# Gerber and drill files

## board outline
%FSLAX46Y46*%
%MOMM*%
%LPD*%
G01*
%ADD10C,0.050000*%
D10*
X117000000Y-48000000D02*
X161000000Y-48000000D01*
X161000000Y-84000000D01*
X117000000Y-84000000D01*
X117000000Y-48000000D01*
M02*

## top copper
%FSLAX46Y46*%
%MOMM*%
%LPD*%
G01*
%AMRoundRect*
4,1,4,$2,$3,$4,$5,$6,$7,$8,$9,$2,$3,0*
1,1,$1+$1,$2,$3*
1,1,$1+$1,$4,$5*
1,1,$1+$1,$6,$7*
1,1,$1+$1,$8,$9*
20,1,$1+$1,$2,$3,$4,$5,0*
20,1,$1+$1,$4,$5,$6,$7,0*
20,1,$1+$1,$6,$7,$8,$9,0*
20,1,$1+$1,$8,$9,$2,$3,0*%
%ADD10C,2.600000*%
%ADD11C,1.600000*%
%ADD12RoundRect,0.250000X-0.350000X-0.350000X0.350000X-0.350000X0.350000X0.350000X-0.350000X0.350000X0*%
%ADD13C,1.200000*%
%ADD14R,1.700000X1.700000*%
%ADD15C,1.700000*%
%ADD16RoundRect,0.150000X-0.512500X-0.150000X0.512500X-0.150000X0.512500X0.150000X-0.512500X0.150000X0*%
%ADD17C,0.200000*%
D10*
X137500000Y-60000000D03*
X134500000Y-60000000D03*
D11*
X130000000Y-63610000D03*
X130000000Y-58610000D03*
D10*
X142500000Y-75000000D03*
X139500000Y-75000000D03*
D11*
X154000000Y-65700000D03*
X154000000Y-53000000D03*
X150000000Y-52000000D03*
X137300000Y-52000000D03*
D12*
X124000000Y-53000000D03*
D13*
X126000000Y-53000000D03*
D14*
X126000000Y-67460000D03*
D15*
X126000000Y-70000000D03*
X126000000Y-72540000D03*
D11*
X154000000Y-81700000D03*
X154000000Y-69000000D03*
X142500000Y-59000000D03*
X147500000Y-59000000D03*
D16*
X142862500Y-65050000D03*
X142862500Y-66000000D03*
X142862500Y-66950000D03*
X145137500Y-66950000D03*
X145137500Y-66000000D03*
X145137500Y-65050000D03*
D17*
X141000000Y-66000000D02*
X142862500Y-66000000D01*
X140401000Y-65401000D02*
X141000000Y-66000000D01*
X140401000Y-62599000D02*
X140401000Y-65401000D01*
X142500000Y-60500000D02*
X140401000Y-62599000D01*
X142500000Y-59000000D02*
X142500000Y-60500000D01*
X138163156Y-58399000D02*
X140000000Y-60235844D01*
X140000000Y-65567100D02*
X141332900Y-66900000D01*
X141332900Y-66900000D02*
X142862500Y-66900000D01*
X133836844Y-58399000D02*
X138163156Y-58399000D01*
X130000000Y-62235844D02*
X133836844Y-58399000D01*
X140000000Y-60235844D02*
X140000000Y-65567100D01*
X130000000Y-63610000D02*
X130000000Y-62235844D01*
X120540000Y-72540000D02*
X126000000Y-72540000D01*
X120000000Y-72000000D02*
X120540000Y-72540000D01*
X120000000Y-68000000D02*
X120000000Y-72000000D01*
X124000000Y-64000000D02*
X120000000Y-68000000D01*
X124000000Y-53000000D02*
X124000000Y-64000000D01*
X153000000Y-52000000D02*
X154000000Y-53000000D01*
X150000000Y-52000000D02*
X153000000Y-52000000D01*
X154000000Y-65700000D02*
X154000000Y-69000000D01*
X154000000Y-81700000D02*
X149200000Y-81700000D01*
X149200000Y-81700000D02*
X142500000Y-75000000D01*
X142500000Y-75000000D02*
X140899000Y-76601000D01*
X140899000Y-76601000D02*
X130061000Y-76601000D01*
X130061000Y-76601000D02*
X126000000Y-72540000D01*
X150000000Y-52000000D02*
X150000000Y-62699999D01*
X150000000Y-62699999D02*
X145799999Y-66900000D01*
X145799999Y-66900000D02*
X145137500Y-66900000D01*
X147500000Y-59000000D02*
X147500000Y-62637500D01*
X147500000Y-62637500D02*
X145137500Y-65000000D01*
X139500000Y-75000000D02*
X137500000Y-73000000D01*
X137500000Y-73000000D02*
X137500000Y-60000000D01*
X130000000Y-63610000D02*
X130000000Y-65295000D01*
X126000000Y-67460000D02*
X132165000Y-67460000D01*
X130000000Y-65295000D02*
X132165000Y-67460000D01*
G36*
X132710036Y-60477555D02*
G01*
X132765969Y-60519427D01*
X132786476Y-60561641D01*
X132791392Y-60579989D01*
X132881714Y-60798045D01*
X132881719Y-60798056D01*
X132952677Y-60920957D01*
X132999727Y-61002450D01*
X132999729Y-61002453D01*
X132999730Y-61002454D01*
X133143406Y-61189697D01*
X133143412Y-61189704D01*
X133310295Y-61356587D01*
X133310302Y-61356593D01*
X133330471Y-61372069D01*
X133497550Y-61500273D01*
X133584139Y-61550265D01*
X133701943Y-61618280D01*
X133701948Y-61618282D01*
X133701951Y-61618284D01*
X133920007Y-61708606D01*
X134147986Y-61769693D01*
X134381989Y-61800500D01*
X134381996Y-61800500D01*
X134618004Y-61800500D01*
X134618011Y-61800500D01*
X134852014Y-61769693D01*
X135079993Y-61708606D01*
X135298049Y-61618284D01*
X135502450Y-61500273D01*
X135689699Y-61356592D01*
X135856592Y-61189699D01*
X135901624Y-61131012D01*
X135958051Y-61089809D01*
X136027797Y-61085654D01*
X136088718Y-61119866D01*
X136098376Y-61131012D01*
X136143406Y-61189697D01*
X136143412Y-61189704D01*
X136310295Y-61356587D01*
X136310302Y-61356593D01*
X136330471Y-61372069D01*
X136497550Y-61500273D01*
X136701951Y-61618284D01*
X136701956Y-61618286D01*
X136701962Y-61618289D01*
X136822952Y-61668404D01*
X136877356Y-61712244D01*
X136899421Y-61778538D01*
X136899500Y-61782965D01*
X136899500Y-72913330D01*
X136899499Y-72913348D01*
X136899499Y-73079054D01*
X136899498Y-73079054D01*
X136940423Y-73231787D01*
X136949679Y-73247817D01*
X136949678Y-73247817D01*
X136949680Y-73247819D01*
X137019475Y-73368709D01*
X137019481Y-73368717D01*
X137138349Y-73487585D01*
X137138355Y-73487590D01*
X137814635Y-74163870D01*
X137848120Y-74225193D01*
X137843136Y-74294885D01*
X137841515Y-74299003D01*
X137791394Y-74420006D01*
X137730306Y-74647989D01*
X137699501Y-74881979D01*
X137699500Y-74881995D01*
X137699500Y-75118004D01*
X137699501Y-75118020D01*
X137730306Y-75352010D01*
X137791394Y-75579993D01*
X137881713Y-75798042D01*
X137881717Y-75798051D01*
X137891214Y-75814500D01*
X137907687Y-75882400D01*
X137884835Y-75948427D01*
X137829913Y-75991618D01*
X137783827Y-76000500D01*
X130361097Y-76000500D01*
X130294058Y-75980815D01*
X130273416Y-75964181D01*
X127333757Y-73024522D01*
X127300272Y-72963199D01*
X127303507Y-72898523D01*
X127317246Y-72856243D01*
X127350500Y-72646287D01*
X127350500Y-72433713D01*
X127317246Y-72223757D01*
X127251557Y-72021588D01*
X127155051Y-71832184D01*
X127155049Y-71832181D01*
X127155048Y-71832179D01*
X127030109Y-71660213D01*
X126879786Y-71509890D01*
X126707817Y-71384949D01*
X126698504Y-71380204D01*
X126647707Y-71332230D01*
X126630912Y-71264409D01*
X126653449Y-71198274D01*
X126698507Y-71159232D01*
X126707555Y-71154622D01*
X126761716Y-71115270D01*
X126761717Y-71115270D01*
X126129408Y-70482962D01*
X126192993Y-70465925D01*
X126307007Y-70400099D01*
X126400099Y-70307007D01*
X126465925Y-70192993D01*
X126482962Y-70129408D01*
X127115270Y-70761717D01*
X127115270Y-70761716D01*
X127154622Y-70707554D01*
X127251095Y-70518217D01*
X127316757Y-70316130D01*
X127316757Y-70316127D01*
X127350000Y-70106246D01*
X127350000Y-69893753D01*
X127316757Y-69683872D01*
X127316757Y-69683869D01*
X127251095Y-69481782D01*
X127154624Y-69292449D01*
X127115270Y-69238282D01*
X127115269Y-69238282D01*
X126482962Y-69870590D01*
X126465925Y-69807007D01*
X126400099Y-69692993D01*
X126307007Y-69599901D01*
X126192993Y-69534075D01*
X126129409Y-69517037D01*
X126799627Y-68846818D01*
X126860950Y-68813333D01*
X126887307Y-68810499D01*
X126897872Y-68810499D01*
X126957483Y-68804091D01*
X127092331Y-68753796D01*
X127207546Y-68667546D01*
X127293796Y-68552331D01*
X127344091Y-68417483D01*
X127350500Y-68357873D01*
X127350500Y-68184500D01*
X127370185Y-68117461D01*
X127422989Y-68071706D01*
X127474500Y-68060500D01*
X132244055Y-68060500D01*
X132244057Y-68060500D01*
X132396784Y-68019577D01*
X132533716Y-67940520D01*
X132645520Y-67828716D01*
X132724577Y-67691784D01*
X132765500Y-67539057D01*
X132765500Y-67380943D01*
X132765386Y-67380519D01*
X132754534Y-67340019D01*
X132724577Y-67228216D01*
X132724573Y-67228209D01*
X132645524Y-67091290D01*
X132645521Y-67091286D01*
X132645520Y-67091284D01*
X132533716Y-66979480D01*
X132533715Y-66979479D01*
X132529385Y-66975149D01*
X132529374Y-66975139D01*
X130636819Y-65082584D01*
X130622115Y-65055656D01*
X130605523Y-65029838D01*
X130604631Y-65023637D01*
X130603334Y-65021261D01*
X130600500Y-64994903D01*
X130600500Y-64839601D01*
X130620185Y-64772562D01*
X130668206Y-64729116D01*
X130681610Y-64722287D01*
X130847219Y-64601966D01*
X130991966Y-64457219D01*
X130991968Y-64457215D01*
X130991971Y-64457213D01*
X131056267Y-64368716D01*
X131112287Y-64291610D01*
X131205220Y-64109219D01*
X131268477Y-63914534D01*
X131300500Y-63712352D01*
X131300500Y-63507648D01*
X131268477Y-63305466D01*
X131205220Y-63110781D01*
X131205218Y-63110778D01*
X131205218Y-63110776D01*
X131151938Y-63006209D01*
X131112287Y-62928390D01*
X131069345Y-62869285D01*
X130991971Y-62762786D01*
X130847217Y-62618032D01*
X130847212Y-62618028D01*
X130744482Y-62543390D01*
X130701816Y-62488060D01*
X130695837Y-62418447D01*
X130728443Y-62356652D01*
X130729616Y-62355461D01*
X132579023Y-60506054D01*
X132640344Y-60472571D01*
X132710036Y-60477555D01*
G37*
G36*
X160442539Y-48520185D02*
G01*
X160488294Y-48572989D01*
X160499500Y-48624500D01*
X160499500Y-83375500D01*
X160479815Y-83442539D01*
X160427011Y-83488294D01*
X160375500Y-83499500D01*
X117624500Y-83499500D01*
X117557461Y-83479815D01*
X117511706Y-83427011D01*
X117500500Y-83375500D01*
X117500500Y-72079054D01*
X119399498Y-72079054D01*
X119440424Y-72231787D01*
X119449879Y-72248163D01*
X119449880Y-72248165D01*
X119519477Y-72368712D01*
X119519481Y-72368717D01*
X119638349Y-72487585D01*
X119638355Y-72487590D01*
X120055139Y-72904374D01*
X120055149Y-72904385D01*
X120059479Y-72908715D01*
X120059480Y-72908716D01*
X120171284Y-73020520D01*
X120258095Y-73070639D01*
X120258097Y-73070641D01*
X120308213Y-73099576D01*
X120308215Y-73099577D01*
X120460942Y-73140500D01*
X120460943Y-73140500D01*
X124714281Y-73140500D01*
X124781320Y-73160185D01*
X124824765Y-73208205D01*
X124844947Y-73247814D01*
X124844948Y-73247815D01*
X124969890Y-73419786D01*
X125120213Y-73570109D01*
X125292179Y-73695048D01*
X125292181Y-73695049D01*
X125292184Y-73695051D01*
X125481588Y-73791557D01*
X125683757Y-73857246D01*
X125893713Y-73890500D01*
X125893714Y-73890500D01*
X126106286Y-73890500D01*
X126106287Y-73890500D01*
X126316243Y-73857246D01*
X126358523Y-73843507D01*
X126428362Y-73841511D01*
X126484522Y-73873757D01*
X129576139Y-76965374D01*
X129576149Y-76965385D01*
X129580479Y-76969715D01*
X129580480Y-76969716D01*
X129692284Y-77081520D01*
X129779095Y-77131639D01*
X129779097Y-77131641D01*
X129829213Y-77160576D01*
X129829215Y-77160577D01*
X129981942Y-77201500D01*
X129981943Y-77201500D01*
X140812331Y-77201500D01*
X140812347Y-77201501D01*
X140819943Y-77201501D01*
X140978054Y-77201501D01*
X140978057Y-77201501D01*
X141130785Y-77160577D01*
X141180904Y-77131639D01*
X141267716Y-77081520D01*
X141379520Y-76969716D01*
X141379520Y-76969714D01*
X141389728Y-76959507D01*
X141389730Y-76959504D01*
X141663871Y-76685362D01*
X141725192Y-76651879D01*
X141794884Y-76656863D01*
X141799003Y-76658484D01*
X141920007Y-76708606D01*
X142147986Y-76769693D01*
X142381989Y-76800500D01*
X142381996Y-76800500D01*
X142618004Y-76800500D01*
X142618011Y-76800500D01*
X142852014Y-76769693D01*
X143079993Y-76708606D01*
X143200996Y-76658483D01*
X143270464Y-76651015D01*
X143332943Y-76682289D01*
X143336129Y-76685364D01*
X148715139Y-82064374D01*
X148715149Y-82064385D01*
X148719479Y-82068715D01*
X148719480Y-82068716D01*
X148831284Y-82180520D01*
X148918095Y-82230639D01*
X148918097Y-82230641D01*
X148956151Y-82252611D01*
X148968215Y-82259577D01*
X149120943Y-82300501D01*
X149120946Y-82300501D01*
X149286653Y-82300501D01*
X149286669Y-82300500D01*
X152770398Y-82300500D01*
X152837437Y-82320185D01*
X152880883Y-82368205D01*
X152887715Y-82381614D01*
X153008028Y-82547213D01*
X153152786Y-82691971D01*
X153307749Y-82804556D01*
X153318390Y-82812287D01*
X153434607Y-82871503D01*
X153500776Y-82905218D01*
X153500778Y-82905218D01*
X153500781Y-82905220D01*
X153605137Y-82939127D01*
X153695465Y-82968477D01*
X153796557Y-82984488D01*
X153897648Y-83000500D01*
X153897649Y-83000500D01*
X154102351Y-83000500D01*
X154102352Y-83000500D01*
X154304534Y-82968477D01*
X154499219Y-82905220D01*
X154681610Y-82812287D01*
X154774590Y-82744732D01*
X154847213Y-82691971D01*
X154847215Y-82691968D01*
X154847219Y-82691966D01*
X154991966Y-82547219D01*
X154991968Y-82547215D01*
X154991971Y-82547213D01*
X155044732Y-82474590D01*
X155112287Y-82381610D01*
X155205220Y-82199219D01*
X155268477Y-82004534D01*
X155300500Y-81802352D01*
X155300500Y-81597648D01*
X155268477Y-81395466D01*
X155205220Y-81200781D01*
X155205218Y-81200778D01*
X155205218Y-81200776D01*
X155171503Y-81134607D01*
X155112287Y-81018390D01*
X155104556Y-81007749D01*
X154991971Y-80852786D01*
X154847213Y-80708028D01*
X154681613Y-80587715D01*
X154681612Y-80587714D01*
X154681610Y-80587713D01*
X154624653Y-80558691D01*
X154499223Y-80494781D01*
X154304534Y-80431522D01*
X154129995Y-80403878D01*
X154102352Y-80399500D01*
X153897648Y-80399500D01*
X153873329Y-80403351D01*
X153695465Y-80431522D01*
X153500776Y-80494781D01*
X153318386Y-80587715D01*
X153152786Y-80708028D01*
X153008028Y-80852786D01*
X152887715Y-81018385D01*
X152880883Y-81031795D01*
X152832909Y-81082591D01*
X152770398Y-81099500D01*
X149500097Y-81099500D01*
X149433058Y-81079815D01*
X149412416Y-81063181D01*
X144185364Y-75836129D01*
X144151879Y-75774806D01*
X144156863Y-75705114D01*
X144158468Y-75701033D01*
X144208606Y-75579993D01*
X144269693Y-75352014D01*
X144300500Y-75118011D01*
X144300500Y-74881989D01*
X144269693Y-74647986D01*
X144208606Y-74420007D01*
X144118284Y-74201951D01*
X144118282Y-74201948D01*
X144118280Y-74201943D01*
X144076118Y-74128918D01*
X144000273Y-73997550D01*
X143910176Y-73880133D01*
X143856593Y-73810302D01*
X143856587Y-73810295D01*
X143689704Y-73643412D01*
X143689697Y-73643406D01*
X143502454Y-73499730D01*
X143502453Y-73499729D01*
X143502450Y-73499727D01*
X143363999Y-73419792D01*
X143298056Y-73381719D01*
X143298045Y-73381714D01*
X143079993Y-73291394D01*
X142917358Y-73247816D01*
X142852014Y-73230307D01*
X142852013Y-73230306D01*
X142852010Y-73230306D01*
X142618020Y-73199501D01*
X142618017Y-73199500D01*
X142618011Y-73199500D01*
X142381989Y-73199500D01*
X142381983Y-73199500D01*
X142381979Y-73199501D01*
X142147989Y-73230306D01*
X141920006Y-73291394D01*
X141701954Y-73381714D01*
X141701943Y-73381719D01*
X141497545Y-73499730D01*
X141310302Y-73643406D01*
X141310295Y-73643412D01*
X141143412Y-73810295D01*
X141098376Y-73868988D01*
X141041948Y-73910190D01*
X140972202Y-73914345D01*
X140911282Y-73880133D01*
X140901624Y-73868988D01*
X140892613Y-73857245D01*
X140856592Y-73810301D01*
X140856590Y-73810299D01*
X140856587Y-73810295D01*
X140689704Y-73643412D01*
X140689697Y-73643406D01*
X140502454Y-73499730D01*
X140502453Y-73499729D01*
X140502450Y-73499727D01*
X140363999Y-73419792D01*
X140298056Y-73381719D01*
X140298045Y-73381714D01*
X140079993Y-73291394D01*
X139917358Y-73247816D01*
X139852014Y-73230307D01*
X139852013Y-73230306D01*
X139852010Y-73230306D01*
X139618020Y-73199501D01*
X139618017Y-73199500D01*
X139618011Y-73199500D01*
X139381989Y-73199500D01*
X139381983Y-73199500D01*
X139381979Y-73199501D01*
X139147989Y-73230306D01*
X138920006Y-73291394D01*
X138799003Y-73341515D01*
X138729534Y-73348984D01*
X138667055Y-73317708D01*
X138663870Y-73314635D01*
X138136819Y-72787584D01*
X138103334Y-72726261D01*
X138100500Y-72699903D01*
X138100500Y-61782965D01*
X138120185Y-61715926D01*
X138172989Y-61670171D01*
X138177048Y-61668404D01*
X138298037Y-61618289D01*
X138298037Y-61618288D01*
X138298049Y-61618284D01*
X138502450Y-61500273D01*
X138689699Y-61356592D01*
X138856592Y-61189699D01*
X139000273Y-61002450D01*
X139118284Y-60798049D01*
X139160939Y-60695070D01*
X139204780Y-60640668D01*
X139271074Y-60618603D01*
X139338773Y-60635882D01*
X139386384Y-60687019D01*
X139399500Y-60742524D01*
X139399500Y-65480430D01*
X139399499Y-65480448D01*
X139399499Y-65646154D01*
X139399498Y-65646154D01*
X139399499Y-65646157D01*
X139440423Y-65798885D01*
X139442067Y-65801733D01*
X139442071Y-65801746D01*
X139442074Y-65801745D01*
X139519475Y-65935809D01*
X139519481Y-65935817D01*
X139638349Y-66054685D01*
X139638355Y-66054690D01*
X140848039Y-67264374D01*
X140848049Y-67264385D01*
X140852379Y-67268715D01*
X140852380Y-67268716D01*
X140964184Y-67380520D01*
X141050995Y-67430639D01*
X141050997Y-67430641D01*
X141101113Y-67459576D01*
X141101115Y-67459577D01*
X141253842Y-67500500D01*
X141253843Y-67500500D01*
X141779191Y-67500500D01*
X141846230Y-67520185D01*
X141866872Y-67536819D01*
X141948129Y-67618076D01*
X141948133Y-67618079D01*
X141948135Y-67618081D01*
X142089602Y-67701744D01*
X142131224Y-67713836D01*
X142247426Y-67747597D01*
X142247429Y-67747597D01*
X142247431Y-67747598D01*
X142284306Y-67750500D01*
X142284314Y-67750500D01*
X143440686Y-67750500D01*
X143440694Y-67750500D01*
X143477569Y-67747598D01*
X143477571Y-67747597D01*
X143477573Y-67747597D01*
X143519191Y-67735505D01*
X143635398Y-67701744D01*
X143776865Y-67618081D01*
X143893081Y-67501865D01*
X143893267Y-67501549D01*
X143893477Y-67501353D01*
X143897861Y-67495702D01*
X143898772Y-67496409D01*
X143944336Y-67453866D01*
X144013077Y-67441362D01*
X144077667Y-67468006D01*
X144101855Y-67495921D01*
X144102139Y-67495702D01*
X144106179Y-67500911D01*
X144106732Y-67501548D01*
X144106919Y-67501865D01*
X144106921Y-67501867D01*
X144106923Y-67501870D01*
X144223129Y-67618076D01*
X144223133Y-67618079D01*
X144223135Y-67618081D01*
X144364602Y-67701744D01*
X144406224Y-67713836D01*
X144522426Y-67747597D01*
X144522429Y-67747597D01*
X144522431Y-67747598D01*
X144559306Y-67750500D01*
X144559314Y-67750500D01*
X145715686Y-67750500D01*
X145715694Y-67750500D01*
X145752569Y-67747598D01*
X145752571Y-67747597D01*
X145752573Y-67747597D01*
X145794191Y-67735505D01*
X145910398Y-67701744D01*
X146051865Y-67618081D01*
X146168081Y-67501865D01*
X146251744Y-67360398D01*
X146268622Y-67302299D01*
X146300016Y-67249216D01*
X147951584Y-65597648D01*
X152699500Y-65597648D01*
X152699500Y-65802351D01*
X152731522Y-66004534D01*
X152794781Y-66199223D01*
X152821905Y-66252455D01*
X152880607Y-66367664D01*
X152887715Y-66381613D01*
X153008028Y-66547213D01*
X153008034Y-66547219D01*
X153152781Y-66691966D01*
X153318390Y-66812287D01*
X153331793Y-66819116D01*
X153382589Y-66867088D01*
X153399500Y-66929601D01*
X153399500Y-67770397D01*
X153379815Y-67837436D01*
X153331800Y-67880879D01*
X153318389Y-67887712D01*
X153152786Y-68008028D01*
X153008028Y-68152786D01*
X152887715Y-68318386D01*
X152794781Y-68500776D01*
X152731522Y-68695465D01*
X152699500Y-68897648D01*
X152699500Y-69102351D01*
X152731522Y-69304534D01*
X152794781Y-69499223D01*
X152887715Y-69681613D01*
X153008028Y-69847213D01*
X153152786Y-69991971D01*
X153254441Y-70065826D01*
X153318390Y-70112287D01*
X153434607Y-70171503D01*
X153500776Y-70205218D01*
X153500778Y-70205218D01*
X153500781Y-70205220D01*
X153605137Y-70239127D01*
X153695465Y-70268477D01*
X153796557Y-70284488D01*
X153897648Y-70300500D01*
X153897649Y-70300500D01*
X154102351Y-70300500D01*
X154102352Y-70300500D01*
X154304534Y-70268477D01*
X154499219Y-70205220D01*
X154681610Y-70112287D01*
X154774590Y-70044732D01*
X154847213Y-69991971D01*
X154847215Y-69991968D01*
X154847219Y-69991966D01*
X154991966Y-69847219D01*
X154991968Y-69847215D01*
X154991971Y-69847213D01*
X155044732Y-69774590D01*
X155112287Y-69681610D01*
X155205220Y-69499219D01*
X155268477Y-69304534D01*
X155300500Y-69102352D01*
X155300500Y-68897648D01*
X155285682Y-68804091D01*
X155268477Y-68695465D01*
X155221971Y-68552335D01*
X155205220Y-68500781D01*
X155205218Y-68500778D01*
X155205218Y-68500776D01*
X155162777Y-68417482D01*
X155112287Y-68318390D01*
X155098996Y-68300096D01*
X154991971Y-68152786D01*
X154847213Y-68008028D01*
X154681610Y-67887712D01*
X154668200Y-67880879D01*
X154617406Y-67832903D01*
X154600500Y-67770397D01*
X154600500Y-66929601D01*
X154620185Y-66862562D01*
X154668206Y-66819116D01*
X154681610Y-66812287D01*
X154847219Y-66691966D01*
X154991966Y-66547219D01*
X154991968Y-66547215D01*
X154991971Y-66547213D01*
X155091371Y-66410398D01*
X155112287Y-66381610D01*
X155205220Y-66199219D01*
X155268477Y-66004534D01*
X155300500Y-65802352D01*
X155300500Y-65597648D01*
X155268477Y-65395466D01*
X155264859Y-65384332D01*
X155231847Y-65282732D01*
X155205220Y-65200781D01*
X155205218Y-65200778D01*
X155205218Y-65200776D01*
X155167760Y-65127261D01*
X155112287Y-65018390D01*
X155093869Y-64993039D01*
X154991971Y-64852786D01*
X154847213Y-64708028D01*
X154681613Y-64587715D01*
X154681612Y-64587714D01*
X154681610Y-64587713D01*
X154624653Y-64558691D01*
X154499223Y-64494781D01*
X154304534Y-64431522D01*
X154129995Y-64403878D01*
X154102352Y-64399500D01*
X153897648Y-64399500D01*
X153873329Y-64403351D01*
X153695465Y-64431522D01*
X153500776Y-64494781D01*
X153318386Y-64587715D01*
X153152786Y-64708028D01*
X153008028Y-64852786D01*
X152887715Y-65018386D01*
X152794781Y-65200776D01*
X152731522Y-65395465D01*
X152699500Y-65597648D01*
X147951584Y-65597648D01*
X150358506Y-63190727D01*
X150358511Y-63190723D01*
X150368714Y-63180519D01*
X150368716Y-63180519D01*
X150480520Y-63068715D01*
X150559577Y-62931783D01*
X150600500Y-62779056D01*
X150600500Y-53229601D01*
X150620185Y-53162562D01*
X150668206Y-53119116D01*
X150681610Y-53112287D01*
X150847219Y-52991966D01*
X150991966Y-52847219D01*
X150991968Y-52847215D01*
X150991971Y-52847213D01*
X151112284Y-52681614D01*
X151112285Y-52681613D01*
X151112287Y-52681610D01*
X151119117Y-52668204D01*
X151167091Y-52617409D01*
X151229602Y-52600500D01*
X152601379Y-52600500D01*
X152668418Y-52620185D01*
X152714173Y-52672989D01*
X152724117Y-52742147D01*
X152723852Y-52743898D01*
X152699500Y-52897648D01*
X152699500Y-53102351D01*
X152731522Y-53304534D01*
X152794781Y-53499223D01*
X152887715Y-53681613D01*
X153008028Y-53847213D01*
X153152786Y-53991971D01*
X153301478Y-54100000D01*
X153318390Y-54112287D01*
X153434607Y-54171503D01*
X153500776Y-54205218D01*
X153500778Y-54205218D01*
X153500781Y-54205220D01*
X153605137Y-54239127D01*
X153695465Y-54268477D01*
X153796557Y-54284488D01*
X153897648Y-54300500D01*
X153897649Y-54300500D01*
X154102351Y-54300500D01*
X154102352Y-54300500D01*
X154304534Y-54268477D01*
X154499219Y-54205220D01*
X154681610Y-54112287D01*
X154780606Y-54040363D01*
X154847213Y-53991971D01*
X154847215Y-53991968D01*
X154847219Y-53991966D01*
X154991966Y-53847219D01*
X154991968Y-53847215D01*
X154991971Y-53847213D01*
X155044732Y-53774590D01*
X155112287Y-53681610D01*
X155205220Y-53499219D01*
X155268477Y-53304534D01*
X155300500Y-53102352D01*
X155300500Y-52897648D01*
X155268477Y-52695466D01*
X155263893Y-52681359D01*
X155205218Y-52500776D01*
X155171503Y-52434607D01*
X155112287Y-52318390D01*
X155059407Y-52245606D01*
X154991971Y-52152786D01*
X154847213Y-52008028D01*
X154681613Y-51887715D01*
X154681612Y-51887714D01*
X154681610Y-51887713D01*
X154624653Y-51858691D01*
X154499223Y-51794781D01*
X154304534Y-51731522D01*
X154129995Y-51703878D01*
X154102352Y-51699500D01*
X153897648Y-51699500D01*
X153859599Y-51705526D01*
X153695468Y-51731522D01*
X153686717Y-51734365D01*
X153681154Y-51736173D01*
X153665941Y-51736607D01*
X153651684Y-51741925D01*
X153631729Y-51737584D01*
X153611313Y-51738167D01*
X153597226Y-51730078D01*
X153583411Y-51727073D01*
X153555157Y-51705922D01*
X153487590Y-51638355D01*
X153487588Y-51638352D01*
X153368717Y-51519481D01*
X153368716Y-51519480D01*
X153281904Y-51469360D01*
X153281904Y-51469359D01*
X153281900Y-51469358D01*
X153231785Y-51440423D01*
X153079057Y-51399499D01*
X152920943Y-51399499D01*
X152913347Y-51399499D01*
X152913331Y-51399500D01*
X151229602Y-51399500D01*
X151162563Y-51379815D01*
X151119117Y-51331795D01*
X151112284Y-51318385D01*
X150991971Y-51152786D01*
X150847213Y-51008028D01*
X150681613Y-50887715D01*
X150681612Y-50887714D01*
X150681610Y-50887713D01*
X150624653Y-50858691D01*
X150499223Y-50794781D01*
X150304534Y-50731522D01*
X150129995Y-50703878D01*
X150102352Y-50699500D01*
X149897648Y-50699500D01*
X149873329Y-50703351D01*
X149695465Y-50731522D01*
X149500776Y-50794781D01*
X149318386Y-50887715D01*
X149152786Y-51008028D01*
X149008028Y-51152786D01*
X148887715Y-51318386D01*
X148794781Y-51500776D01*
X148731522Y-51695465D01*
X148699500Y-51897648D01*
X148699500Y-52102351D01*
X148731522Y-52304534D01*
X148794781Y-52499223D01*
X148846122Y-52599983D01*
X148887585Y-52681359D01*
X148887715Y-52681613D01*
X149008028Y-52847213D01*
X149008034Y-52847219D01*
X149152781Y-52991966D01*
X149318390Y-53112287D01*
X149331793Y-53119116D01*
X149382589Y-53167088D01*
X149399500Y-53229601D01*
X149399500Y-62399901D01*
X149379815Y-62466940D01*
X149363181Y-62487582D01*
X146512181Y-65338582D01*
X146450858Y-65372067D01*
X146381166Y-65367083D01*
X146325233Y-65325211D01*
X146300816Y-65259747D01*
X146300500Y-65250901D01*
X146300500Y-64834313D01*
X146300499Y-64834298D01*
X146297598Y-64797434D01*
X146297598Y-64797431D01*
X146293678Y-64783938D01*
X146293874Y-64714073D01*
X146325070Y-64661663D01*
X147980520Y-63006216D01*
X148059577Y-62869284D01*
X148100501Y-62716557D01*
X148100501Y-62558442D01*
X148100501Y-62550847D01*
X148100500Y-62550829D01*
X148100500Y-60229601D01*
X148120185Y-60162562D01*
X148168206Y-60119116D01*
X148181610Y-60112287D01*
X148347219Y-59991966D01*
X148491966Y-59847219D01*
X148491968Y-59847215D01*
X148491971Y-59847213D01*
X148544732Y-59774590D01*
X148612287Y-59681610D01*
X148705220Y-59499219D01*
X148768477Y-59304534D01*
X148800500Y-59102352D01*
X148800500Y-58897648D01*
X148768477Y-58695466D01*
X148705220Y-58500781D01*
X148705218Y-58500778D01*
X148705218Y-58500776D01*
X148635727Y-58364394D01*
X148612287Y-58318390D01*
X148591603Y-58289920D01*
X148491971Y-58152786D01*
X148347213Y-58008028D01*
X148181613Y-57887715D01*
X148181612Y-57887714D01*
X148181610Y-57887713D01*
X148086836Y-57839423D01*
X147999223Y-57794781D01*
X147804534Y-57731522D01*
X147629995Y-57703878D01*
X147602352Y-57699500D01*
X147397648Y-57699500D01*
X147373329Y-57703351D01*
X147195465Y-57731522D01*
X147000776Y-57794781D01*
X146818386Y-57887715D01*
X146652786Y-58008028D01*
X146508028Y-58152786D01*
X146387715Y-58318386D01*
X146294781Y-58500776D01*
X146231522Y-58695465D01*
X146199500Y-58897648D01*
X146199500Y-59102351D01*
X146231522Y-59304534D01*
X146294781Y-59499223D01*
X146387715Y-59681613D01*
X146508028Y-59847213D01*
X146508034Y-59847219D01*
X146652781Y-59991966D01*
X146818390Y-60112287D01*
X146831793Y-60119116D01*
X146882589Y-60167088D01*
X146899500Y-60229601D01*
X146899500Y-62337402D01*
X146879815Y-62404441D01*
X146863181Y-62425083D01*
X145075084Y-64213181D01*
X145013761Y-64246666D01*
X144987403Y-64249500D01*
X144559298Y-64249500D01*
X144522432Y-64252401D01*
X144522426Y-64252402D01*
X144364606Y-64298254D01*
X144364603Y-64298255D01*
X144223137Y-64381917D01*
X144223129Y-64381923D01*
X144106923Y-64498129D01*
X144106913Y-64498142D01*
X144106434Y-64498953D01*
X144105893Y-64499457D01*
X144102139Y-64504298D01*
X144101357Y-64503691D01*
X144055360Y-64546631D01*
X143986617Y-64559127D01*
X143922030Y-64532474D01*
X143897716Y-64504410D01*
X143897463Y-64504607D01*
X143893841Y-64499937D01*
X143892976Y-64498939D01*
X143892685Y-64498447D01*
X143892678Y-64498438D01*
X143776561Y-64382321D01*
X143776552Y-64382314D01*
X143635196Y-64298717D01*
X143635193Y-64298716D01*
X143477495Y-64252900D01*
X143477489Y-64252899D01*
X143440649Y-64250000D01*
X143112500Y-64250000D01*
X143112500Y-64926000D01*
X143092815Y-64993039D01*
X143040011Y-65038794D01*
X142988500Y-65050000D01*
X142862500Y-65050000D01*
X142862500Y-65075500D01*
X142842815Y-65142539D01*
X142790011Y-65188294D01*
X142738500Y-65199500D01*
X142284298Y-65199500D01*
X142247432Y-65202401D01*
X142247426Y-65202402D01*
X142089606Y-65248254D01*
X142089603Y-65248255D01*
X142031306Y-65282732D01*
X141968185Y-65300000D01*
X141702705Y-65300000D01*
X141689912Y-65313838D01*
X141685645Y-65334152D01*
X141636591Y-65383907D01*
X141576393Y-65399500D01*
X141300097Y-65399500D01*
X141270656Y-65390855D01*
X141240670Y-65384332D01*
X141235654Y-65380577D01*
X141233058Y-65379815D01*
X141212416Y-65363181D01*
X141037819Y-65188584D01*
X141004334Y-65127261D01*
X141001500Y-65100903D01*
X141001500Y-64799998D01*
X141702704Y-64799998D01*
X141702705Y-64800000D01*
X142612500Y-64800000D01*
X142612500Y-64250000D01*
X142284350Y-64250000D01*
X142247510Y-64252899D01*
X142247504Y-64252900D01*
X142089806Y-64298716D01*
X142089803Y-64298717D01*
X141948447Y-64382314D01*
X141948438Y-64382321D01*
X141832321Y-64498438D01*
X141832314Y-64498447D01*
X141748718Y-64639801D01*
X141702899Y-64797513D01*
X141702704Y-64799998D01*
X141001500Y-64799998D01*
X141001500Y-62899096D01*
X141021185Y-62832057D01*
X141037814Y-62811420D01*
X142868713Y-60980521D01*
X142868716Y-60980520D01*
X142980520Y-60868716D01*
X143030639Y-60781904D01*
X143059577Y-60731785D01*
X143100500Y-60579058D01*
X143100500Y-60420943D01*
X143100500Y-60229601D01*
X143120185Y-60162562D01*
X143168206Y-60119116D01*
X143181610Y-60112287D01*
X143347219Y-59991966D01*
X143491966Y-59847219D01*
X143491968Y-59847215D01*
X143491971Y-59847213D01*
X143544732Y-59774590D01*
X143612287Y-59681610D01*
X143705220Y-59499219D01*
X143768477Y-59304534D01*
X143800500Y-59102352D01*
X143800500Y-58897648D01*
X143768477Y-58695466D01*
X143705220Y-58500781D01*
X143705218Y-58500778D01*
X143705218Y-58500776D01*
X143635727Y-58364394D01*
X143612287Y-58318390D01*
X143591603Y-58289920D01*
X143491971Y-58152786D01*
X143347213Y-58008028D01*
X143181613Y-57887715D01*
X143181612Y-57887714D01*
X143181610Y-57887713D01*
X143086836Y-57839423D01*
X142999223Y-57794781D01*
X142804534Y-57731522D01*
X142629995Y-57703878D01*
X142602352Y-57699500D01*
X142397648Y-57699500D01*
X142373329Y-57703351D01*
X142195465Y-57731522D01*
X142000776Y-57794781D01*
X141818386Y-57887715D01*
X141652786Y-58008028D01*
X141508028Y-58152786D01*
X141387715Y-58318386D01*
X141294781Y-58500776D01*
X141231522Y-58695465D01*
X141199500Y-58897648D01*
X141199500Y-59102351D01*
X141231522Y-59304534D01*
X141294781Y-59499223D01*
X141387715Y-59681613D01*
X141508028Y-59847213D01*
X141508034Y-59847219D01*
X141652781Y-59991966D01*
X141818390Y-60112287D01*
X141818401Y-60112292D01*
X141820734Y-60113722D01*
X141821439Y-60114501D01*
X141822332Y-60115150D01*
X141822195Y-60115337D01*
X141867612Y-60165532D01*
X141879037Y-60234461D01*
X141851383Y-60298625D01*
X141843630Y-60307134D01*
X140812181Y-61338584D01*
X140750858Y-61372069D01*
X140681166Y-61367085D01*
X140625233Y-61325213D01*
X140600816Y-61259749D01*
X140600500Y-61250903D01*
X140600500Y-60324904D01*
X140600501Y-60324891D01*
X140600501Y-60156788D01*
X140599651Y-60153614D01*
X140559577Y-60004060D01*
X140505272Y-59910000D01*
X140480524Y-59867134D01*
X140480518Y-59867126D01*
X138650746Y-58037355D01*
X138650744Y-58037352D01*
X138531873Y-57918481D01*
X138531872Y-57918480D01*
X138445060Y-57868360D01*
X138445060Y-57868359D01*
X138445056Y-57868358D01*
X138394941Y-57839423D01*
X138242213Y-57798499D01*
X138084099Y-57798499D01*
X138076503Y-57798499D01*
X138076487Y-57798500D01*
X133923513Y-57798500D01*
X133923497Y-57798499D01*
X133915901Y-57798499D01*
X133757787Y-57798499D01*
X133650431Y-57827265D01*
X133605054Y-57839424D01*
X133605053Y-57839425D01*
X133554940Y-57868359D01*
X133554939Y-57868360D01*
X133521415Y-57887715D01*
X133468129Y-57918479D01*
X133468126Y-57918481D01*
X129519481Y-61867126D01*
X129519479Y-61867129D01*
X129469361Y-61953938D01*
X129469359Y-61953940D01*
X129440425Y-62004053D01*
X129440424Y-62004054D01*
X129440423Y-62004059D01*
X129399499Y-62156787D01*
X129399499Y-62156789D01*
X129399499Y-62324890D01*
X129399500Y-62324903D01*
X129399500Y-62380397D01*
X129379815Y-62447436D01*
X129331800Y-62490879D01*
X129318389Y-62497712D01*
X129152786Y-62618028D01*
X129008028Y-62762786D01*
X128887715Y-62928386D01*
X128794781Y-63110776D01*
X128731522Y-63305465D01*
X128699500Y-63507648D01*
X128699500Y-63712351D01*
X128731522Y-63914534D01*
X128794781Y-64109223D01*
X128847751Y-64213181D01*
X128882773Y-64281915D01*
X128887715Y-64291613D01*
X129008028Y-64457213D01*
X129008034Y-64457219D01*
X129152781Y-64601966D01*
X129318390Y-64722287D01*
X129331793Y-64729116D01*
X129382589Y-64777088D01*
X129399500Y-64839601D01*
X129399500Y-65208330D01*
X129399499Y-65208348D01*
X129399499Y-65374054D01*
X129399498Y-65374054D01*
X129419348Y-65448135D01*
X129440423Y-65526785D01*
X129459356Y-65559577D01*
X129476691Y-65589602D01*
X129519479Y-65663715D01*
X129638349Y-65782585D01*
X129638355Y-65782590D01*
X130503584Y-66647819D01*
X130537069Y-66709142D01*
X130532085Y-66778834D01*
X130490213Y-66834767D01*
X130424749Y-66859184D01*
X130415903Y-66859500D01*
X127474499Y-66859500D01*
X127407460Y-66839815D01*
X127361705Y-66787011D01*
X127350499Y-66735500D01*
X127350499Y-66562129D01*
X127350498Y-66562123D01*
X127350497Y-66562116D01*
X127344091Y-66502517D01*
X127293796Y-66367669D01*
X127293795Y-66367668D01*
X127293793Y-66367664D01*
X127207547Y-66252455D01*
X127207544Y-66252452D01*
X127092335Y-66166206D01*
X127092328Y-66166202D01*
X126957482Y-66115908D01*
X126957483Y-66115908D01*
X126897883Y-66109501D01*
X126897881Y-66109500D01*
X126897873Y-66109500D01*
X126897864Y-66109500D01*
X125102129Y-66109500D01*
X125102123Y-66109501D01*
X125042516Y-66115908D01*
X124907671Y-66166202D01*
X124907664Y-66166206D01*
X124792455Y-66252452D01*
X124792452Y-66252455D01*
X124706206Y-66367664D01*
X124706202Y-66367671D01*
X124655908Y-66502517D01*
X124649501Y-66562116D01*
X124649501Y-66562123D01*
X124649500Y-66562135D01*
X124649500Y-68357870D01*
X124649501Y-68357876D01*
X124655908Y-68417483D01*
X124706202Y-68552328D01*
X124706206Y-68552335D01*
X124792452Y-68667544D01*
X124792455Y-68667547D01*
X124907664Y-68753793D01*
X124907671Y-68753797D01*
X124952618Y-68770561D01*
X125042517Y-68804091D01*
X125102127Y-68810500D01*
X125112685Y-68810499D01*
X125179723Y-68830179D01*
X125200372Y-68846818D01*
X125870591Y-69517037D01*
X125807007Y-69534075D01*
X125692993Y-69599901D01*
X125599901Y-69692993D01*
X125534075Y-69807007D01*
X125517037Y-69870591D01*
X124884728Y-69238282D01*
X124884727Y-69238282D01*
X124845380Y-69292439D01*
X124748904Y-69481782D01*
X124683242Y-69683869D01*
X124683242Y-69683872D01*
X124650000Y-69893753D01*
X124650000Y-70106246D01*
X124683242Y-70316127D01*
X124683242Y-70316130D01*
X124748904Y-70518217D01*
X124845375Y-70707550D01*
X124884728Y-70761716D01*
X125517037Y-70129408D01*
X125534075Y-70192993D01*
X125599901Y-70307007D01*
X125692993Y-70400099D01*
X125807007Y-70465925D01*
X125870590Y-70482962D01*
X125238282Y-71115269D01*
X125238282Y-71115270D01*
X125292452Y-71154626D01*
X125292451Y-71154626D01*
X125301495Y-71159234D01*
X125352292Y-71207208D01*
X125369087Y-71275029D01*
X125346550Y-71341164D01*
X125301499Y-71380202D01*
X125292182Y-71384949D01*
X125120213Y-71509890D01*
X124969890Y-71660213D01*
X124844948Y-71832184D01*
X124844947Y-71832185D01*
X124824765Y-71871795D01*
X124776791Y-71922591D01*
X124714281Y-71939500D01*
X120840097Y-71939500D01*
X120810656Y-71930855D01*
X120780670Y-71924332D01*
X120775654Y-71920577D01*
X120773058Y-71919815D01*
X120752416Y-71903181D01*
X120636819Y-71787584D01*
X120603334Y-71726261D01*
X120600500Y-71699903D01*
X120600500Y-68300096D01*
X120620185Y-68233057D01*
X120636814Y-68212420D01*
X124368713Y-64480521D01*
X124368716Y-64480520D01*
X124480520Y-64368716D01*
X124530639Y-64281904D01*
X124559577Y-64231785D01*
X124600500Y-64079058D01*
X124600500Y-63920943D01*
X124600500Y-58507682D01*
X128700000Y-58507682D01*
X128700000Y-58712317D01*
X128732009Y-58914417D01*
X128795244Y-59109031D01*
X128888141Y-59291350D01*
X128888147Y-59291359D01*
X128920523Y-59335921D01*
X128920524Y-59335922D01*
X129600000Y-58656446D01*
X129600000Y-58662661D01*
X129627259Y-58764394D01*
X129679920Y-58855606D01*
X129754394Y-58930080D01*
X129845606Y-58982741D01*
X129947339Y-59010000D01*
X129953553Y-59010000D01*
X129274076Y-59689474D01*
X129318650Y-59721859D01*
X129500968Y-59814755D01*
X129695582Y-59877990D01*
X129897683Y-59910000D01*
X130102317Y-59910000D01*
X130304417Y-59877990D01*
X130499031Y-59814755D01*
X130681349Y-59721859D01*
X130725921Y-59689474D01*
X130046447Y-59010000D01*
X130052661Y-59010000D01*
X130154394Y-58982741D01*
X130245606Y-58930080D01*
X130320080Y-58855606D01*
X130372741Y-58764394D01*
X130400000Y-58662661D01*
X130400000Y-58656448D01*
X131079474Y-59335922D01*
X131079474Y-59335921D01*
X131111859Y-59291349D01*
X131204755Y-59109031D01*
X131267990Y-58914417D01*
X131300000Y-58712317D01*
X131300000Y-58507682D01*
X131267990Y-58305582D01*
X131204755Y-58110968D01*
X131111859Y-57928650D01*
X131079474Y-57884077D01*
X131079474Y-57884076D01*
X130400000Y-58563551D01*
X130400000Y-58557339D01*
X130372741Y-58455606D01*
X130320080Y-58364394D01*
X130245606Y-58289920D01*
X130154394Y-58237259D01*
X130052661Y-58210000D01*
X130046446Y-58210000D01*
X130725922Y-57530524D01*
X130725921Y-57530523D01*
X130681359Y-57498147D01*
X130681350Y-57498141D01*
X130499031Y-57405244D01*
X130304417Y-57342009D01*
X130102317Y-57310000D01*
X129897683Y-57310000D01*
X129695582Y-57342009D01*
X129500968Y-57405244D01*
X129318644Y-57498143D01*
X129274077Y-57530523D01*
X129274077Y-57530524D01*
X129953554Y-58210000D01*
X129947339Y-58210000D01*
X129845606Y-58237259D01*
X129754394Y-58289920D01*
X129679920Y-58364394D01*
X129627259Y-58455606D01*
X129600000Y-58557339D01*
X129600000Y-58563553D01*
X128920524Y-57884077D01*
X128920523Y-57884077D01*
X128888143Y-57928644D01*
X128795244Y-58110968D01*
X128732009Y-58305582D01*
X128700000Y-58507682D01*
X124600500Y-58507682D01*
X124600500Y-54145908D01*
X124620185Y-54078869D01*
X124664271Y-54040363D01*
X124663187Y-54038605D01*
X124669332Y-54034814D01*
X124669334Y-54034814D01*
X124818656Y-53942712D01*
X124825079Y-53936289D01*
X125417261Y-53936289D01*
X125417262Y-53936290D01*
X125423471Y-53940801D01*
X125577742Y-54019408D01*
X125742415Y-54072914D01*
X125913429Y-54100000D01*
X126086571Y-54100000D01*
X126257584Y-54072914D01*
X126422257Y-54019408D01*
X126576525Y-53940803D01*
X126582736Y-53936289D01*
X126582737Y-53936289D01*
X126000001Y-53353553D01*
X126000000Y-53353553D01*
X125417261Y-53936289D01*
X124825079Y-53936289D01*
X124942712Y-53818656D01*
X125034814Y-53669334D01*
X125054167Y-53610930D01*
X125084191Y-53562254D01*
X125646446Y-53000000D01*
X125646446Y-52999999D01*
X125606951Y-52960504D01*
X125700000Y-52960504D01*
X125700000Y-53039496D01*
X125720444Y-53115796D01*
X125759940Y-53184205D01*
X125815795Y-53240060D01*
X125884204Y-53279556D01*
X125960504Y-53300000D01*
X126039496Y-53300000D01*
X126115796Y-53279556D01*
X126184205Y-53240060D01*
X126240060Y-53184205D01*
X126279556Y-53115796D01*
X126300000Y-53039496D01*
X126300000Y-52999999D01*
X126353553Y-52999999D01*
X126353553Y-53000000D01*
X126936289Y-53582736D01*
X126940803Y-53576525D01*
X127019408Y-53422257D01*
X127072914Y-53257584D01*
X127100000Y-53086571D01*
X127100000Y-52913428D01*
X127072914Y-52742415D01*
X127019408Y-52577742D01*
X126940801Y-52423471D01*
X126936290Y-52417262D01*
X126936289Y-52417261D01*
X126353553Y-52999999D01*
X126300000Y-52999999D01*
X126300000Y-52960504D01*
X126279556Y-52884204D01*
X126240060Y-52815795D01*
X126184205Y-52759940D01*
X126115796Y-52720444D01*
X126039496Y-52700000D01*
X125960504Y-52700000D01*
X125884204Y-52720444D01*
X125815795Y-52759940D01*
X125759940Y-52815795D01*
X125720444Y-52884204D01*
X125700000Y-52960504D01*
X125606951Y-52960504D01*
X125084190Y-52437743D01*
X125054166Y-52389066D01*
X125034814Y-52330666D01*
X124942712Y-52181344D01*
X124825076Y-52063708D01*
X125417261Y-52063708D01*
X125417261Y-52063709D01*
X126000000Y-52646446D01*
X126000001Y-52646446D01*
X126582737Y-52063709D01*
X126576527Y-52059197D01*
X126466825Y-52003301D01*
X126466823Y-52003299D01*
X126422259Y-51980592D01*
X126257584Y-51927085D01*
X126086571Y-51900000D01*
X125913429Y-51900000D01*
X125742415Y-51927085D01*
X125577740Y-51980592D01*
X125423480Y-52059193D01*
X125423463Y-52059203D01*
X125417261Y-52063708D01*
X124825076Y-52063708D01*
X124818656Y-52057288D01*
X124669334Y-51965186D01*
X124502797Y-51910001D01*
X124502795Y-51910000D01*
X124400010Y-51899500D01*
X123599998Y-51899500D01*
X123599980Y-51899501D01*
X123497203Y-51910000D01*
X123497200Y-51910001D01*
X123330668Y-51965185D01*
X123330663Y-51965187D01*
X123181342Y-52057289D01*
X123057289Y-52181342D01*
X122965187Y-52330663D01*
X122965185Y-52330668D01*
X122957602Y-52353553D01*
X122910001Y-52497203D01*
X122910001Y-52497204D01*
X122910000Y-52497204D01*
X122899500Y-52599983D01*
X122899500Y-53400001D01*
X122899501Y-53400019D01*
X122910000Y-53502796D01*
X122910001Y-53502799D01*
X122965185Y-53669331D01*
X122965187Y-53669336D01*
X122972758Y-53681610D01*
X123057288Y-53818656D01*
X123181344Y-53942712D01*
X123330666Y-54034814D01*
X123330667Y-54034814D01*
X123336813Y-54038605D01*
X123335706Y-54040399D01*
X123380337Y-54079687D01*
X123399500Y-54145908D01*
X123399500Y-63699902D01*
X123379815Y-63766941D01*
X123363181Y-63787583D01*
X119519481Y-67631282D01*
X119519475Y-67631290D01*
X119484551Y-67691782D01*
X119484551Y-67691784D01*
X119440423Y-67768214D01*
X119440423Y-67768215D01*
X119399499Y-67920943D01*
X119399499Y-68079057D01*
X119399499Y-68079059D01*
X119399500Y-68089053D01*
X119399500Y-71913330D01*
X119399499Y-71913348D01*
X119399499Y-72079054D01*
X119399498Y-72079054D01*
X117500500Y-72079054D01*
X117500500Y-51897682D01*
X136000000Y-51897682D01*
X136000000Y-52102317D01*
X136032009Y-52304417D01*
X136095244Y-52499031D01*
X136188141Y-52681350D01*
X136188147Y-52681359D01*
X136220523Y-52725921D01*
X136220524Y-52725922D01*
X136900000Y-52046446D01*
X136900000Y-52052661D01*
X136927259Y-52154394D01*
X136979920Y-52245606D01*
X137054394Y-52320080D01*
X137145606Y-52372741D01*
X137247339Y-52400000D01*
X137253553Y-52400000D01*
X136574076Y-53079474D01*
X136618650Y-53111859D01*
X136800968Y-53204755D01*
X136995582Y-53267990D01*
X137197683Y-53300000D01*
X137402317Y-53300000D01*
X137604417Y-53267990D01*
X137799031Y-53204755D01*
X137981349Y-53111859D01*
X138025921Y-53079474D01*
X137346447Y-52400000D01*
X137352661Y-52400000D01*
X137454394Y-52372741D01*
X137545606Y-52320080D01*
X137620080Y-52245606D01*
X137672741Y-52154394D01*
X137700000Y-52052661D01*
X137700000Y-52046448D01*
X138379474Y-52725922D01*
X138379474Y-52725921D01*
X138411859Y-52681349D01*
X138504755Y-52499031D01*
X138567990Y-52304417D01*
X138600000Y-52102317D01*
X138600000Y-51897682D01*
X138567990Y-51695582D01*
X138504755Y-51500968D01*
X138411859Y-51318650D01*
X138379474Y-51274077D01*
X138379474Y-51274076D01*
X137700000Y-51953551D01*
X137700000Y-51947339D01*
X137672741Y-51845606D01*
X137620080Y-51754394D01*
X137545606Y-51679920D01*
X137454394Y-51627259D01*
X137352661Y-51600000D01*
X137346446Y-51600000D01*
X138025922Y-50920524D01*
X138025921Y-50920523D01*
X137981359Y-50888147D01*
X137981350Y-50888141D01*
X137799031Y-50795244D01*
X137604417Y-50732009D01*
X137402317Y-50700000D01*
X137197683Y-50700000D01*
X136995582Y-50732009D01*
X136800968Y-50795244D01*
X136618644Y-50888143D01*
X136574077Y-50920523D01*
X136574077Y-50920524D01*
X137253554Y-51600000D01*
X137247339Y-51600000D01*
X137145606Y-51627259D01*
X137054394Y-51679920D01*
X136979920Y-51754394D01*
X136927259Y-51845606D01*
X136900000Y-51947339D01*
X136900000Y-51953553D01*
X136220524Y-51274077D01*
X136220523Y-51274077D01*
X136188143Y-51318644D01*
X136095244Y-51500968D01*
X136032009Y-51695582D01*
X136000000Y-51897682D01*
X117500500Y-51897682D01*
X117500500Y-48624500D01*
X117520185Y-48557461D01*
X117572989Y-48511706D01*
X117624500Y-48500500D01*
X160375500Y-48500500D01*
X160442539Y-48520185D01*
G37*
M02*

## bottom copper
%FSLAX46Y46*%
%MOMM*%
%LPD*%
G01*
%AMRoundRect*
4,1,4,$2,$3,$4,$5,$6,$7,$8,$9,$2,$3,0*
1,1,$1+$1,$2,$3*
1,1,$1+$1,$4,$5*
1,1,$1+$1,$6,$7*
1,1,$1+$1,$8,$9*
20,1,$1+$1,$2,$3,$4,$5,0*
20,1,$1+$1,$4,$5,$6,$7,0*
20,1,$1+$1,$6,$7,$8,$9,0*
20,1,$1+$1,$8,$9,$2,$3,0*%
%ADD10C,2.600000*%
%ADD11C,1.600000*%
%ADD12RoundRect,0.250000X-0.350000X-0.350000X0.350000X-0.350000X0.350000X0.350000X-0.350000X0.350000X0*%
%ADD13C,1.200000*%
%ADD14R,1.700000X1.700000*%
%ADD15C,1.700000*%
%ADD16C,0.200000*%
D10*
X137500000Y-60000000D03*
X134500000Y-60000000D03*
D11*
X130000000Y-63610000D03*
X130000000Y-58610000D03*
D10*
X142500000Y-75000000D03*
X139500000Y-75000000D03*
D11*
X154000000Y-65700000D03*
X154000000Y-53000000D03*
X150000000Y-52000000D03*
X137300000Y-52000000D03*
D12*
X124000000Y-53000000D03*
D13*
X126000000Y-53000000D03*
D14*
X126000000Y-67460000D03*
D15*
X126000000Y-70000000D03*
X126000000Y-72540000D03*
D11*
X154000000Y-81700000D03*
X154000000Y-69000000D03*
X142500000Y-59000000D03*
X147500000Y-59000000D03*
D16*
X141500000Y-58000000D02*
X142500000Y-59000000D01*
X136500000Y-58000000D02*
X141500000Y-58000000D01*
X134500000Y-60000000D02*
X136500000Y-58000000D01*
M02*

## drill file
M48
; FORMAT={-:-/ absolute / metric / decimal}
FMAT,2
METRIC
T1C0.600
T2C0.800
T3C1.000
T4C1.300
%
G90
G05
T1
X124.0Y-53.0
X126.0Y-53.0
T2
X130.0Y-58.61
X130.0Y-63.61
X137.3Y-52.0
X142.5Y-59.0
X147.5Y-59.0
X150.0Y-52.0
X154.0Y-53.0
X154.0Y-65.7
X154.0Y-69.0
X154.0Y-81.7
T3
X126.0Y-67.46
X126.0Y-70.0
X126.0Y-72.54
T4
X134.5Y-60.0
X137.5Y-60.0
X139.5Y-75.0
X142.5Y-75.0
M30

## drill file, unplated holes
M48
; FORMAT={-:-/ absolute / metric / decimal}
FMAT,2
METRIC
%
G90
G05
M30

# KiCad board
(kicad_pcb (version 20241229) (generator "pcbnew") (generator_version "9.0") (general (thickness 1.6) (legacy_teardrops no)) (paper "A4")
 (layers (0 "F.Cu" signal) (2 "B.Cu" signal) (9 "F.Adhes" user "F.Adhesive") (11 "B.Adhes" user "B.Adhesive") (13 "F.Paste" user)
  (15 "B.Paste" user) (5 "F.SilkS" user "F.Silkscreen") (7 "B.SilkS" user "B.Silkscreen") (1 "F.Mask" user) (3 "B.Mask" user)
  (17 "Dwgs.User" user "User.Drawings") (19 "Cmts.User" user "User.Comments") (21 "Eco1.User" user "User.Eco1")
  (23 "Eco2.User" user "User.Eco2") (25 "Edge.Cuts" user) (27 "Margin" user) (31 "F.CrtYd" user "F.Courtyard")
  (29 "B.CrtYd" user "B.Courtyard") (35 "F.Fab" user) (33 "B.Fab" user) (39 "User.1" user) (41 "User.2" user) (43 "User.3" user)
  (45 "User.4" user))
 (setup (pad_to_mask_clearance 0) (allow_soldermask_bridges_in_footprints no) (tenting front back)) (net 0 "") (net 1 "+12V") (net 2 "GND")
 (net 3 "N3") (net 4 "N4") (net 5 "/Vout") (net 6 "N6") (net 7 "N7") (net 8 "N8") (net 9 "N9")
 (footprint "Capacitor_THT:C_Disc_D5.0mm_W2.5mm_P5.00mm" (layer "F.Cu") (at 130 63.61 90)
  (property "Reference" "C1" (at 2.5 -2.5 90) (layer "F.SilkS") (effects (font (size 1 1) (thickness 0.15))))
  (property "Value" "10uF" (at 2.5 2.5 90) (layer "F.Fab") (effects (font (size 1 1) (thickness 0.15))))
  (pad "1" thru_hole circle (at 0 0 90) (size 1.6 1.6) (drill 0.8) (layers "*.Cu" "*.Mask") (remove_unused_layers no) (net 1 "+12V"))
  (pad "2" thru_hole circle (at 5 0 90) (size 1.6 1.6) (drill 0.8) (layers "*.Cu" "*.Mask") (remove_unused_layers no) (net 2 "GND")))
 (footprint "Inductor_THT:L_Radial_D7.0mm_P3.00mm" (layer "F.Cu") (at 134.5 60)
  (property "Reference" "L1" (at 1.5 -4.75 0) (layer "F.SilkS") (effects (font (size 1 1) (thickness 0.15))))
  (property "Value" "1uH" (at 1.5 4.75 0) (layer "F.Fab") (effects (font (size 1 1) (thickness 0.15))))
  (pad "1" thru_hole circle (at 0 0) (size 2.6 2.6) (drill 1.3) (layers "*.Cu" "*.Mask") (remove_unused_layers no) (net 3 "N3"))
  (pad "2" thru_hole circle (at 3 0) (size 2.6 2.6) (drill 1.3) (layers "*.Cu" "*.Mask") (remove_unused_layers no) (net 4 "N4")))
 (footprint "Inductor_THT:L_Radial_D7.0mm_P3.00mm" (layer "F.Cu") (at 139.5 75)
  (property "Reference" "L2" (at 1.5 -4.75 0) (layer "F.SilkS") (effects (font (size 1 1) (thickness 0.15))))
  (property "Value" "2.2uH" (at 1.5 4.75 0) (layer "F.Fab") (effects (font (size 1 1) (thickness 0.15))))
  (pad "1" thru_hole circle (at 0 0) (size 2.6 2.6) (drill 1.3) (layers "*.Cu" "*.Mask") (remove_unused_layers no) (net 4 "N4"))
  (pad "2" thru_hole circle (at 3 0) (size 2.6 2.6) (drill 1.3) (layers "*.Cu" "*.Mask") (remove_unused_layers no) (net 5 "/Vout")))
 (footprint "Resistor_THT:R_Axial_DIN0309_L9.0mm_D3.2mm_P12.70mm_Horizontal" (layer "F.Cu") (at 154 65.7 90)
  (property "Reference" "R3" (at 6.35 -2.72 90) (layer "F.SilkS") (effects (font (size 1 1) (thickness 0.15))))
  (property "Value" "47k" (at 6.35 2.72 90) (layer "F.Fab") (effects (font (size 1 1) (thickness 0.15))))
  (pad "1" thru_hole circle (at 0 0 90) (size 1.6 1.6) (drill 0.8) (layers "*.Cu" "*.Mask") (remove_unused_layers no) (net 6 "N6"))
  (pad "2" thru_hole circle (at 12.7 0 90) (size 1.6 1.6) (drill 0.8) (layers "*.Cu" "*.Mask") (remove_unused_layers no) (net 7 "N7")))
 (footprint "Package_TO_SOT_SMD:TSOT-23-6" (layer "F.Cu") (at 144 66)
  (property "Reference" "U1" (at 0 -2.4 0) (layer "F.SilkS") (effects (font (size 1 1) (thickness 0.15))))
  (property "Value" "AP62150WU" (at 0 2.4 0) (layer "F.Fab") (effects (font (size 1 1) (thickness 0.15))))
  (pad "1" smd roundrect (at -1.1375 -0.95) (size 1.325 0.6) (layers "F.Cu" "F.Mask" "F.Paste") (roundrect_rratio 0.25) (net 2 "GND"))
  (pad "2" smd roundrect (at -1.1375 0) (size 1.325 0.6) (layers "F.Cu" "F.Mask" "F.Paste") (roundrect_rratio 0.25) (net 3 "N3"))
  (pad "3" smd roundrect (at -1.1375 0.95) (size 1.325 0.6) (layers "F.Cu" "F.Mask" "F.Paste") (roundrect_rratio 0.25) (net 1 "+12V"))
  (pad "4" smd roundrect (at 1.1375 0.95) (size 1.325 0.6) (layers "F.Cu" "F.Mask" "F.Paste") (roundrect_rratio 0.25) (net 7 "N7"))
  (pad "5" smd roundrect (at 1.1375 0) (size 1.325 0.6) (layers "F.Cu" "F.Mask" "F.Paste") (roundrect_rratio 0.25) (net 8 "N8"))
  (pad "6" smd roundrect (at 1.1375 -0.95) (size 1.325 0.6) (layers "F.Cu" "F.Mask" "F.Paste") (roundrect_rratio 0.25) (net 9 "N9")))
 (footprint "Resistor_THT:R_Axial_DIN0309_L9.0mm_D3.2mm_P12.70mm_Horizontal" (layer "F.Cu") (at 150 52 180)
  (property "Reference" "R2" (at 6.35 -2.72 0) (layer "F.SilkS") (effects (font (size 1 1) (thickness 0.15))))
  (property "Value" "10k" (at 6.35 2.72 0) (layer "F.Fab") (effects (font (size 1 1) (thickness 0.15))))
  (pad "1" thru_hole circle (at 0 0 180) (size 1.6 1.6) (drill 0.8) (layers "*.Cu" "*.Mask") (remove_unused_layers no) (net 7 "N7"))
  (pad "2" thru_hole circle (at 12.7 0 180) (size 1.6 1.6) (drill 0.8) (layers "*.Cu" "*.Mask") (remove_unused_layers no) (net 2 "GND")))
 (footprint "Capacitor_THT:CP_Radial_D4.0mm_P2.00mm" (layer "F.Cu") (at 124 53)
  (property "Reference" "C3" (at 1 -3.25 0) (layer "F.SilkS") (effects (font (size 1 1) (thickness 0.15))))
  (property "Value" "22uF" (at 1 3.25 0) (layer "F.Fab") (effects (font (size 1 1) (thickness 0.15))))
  (pad "1" thru_hole roundrect (at 0 0) (size 1.2 1.2) (drill 0.6) (layers "*.Cu" "*.Mask") (remove_unused_layers no)
   (roundrect_rratio 0.208333) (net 5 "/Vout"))
  (pad "2" thru_hole circle (at 2 0) (size 1.2 1.2) (drill 0.6) (layers "*.Cu" "*.Mask") (remove_unused_layers no) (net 2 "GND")))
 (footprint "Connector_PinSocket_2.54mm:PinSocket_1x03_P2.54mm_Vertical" (layer "F.Cu") (at 126 67.46)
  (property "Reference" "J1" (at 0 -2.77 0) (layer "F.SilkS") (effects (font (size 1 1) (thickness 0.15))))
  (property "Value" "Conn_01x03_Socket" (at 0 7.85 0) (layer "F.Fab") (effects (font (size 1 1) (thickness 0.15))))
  (pad "1" thru_hole rect (at 0 0) (size 1.7 1.7) (drill 1) (layers "*.Cu" "*.Mask") (remove_unused_layers no) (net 1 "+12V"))
  (pad "2" thru_hole circle (at 0 2.54) (size 1.7 1.7) (drill 1) (layers "*.Cu" "*.Mask") (remove_unused_layers no) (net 2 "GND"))
  (pad "3" thru_hole circle (at 0 5.08) (size 1.7 1.7) (drill 1) (layers "*.Cu" "*.Mask") (remove_unused_layers no) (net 5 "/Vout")))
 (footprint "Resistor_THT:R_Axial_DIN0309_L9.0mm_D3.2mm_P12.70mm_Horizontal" (layer "F.Cu") (at 154 81.7 90)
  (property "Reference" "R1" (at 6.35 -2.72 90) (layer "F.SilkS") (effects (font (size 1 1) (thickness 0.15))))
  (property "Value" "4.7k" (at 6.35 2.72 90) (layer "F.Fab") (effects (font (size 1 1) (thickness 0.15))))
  (pad "1" thru_hole circle (at 0 0 90) (size 1.6 1.6) (drill 0.8) (layers "*.Cu" "*.Mask") (remove_unused_layers no) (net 5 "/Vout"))
  (pad "2" thru_hole circle (at 12.7 0 90) (size 1.6 1.6) (drill 0.8) (layers "*.Cu" "*.Mask") (remove_unused_layers no) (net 6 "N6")))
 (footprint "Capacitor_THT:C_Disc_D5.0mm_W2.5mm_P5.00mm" (layer "F.Cu") (at 142.5 59)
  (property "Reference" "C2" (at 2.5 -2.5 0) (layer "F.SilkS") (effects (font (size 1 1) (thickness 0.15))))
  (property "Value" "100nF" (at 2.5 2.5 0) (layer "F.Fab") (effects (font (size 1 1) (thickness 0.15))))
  (pad "1" thru_hole circle (at 0 0) (size 1.6 1.6) (drill 0.8) (layers "*.Cu" "*.Mask") (remove_unused_layers no) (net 3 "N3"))
  (pad "2" thru_hole circle (at 5 0) (size 1.6 1.6) (drill 0.8) (layers "*.Cu" "*.Mask") (remove_unused_layers no) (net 9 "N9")))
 (gr_rect (start 117 48) (end 161 84) (stroke (width 0.05) (type default)) (fill no) (layer "Edge.Cuts"))
 (segment (start 138.163156 58.399) (end 140 60.235844) (width 0.2) (layer "F.Cu") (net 1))
 (segment (start 130 65.295) (end 132.165 67.46) (width 0.2) (layer "F.Cu") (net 1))
 (segment (start 130 63.61) (end 130 62.235844) (width 0.2) (layer "F.Cu") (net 1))
 (segment (start 130 63.61) (end 130 65.295) (width 0.2) (layer "F.Cu") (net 1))
 (segment (start 141.3329 66.9) (end 142.8625 66.9) (width 0.2) (layer "F.Cu") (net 1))
 (segment (start 140 60.235844) (end 140 65.5671) (width 0.2) (layer "F.Cu") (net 1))
 (segment (start 133.836844 58.399) (end 138.163156 58.399) (width 0.2) (layer "F.Cu") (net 1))
 (segment (start 140 65.5671) (end 141.3329 66.9) (width 0.2) (layer "F.Cu") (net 1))
 (segment (start 130 62.235844) (end 133.836844 58.399) (width 0.2) (layer "F.Cu") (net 1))
 (segment (start 126 67.46) (end 132.165 67.46) (width 0.2) (layer "F.Cu") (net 1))
 (segment (start 140.401 65.401) (end 141 66) (width 0.2) (layer "F.Cu") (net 3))
 (segment (start 141 66) (end 142.8625 66) (width 0.2) (layer "F.Cu") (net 3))
 (segment (start 142.5 59) (end 142.5 60.5) (width 0.2) (layer "F.Cu") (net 3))
 (segment (start 140.401 62.599) (end 140.401 65.401) (width 0.2) (layer "F.Cu") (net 3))
 (segment (start 142.5 60.5) (end 140.401 62.599) (width 0.2) (layer "F.Cu") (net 3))
 (segment (start 136.5 58) (end 141.5 58) (width 0.2) (layer "B.Cu") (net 3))
 (segment (start 134.5 60) (end 136.5 58) (width 0.2) (layer "B.Cu") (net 3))
 (segment (start 141.5 58) (end 142.5 59) (width 0.2) (layer "B.Cu") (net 3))
 (segment (start 147.5 59) (end 147.5 62.6375) (width 0.2) (layer "F.Cu") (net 9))
 (segment (start 147.5 62.6375) (end 145.1375 65) (width 0.2) (layer "F.Cu") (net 9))
 (segment (start 130.061 76.601) (end 126 72.54) (width 0.2) (layer "F.Cu") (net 5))
 (segment (start 149.2 81.7) (end 142.5 75) (width 0.2) (layer "F.Cu") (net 5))
 (segment (start 120 72) (end 120.54 72.54) (width 0.2) (layer "F.Cu") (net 5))
 (segment (start 154 81.7) (end 149.2 81.7) (width 0.2) (layer "F.Cu") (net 5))
 (segment (start 124 53) (end 124 64) (width 0.2) (layer "F.Cu") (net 5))
 (segment (start 120 68) (end 120 72) (width 0.2) (layer "F.Cu") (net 5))
 (segment (start 142.5 75) (end 140.899 76.601) (width 0.2) (layer "F.Cu") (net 5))
 (segment (start 124 64) (end 120 68) (width 0.2) (layer "F.Cu") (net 5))
 (segment (start 140.899 76.601) (end 130.061 76.601) (width 0.2) (layer "F.Cu") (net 5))
 (segment (start 120.54 72.54) (end 126 72.54) (width 0.2) (layer "F.Cu") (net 5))
 (segment (start 139.5 75) (end 137.5 73) (width 0.2) (layer "F.Cu") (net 4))
 (segment (start 137.5 73) (end 137.5 60) (width 0.2) (layer "F.Cu") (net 4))
 (segment (start 154 65.7) (end 154 69) (width 0.2) (layer "F.Cu") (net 6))
 (segment (start 150 52) (end 150 62.699999) (width 0.2) (layer "F.Cu") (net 7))
 (segment (start 145.799999 66.9) (end 145.1375 66.9) (width 0.2) (layer "F.Cu") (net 7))
 (segment (start 150 62.699999) (end 145.799999 66.9) (width 0.2) (layer "F.Cu") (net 7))
 (segment (start 153 52) (end 154 53) (width 0.2) (layer "F.Cu") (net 7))
 (segment (start 150 52) (end 153 52) (width 0.2) (layer "F.Cu") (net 7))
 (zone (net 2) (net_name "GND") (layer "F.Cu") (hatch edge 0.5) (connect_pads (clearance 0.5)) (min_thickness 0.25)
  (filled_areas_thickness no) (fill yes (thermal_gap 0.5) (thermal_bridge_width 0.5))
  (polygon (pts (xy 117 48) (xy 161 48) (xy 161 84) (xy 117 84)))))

